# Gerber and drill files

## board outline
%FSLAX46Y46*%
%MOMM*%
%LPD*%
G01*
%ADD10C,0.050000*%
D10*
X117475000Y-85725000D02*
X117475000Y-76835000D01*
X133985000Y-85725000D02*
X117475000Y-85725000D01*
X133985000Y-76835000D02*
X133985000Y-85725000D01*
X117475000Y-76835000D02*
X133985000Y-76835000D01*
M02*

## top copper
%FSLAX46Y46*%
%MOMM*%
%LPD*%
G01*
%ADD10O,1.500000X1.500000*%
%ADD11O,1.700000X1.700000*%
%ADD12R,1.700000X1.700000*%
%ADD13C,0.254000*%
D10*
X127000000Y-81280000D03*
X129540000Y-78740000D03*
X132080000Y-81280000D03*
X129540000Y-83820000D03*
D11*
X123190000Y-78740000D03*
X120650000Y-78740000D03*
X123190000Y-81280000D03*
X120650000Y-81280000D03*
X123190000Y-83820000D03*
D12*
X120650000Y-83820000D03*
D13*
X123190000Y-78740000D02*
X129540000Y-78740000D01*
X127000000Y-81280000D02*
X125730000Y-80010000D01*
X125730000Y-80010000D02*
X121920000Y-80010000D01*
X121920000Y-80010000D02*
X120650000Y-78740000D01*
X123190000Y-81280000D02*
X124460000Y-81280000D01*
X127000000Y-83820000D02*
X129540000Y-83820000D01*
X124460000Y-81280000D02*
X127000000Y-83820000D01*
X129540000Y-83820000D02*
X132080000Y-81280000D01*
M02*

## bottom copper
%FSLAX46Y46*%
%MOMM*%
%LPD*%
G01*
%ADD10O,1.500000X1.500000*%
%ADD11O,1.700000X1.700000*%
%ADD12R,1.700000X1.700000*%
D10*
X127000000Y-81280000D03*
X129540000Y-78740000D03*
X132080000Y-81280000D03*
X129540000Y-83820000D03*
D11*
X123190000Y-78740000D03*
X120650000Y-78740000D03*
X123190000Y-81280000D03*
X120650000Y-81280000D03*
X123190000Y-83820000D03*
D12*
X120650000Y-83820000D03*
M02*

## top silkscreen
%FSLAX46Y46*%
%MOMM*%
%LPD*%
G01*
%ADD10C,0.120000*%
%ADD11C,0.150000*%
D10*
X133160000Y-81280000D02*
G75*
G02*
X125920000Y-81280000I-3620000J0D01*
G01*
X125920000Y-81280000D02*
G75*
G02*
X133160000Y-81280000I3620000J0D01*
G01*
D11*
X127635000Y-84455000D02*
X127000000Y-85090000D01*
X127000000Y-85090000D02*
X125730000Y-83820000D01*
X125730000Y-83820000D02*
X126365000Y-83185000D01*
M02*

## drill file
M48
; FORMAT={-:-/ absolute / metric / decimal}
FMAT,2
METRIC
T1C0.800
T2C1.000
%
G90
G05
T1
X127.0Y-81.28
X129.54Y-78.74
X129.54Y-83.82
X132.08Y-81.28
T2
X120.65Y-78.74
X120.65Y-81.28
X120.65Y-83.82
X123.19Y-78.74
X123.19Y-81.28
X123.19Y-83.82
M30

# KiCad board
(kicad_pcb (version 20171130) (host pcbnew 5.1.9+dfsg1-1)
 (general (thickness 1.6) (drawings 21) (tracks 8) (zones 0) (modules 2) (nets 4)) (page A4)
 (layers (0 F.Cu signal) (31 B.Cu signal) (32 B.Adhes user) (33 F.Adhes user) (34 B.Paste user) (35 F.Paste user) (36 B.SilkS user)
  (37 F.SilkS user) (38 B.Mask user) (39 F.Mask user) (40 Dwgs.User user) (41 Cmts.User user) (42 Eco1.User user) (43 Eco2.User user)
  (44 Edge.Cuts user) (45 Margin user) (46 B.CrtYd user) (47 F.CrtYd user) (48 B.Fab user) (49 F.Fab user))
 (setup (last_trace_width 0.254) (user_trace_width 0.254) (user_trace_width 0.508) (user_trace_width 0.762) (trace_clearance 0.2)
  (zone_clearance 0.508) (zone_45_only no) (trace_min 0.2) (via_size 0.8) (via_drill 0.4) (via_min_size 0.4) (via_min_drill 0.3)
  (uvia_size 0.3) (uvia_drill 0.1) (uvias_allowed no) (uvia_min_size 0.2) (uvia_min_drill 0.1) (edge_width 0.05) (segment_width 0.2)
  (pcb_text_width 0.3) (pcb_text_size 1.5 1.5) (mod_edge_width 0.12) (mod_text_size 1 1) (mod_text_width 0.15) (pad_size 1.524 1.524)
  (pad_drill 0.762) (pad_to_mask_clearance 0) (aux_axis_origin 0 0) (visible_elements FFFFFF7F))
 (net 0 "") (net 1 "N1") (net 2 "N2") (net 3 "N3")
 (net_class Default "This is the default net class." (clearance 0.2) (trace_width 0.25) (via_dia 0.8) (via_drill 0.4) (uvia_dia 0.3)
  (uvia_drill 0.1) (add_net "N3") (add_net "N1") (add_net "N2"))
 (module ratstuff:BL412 (layer F.Cu) (at 129.54 81.28 180)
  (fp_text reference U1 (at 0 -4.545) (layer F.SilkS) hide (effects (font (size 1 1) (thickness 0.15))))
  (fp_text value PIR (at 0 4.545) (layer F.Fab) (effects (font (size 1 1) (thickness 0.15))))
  (fp_circle (center 0 0) (end 0 3.62) (layer F.SilkS) (width 0.12))
  (fp_line (start 1.905 -3.175) (end 2.54 -3.81) (layer F.SilkS) (width 0.15))
  (fp_line (start 2.54 -3.81) (end 3.81 -2.54) (layer F.SilkS) (width 0.15))
  (fp_line (start 3.81 -2.54) (end 3.175 -1.905) (layer F.SilkS) (width 0.15))
  (pad 4 thru_hole oval (at 2.54 0 180) (size 1.5 1.5) (drill 0.8) (layers *.Cu *.Mask) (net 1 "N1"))
  (pad 3 thru_hole oval (at 0 2.54 180) (size 1.5 1.5) (drill 0.8) (layers *.Cu *.Mask) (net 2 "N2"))
  (pad 2 thru_hole oval (at -2.54 0 180) (size 1.5 1.5) (drill 0.8) (layers *.Cu *.Mask) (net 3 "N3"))
  (pad 1 thru_hole oval (at 0 -2.54 180) (size 1.5 1.5) (drill 0.8) (layers *.Cu *.Mask) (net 3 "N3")))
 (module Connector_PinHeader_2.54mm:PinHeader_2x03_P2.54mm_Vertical (layer B.Cu) (at 120.65 83.82)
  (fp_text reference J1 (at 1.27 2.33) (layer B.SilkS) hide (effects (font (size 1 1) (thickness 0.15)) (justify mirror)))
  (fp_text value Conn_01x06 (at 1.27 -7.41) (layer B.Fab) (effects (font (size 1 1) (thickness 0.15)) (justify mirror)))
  (pad 6 thru_hole oval (at 2.54 -5.08) (size 1.7 1.7) (drill 1) (layers *.Cu *.Mask) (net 2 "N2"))
  (pad 5 thru_hole oval (at 0 -5.08) (size 1.7 1.7) (drill 1) (layers *.Cu *.Mask) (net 1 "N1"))
  (pad 4 thru_hole oval (at 2.54 -2.54) (size 1.7 1.7) (drill 1) (layers *.Cu *.Mask) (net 3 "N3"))
  (pad 3 thru_hole oval (at 0 -2.54) (size 1.7 1.7) (drill 1) (layers *.Cu *.Mask))
  (pad 2 thru_hole oval (at 2.54 0) (size 1.7 1.7) (drill 1) (layers *.Cu *.Mask))
  (pad 1 thru_hole rect (at 0 0) (size 1.7 1.7) (drill 1) (layers *.Cu *.Mask)))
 (gr_line (start 117.475 85.725) (end 117.475 76.835) (layer Edge.Cuts) (width 0.05))
 (gr_line (start 133.985 85.725) (end 117.475 85.725) (layer Edge.Cuts) (width 0.05))
 (gr_line (start 133.985 76.835) (end 133.985 85.725) (layer Edge.Cuts) (width 0.05))
 (gr_line (start 117.475 76.835) (end 133.985 76.835) (layer Edge.Cuts) (width 0.05))
 (segment (start 123.19 78.74) (end 129.54 78.74) (width 0.254) (layer F.Cu) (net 2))
 (segment (start 127 81.28) (end 125.73 80.01) (width 0.254) (layer F.Cu) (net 1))
 (segment (start 125.73 80.01) (end 121.92 80.01) (width 0.254) (layer F.Cu) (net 1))
 (segment (start 121.92 80.01) (end 120.65 78.74) (width 0.254) (layer F.Cu) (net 1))
 (segment (start 123.19 81.28) (end 124.46 81.28) (width 0.254) (layer F.Cu) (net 3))
 (segment (start 127 83.82) (end 129.54 83.82) (width 0.254) (layer F.Cu) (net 3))
 (segment (start 124.46 81.28) (end 127 83.82) (width 0.254) (layer F.Cu) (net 3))
 (segment (start 129.54 83.82) (end 132.08 81.28) (width 0.254) (layer F.Cu) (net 3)))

